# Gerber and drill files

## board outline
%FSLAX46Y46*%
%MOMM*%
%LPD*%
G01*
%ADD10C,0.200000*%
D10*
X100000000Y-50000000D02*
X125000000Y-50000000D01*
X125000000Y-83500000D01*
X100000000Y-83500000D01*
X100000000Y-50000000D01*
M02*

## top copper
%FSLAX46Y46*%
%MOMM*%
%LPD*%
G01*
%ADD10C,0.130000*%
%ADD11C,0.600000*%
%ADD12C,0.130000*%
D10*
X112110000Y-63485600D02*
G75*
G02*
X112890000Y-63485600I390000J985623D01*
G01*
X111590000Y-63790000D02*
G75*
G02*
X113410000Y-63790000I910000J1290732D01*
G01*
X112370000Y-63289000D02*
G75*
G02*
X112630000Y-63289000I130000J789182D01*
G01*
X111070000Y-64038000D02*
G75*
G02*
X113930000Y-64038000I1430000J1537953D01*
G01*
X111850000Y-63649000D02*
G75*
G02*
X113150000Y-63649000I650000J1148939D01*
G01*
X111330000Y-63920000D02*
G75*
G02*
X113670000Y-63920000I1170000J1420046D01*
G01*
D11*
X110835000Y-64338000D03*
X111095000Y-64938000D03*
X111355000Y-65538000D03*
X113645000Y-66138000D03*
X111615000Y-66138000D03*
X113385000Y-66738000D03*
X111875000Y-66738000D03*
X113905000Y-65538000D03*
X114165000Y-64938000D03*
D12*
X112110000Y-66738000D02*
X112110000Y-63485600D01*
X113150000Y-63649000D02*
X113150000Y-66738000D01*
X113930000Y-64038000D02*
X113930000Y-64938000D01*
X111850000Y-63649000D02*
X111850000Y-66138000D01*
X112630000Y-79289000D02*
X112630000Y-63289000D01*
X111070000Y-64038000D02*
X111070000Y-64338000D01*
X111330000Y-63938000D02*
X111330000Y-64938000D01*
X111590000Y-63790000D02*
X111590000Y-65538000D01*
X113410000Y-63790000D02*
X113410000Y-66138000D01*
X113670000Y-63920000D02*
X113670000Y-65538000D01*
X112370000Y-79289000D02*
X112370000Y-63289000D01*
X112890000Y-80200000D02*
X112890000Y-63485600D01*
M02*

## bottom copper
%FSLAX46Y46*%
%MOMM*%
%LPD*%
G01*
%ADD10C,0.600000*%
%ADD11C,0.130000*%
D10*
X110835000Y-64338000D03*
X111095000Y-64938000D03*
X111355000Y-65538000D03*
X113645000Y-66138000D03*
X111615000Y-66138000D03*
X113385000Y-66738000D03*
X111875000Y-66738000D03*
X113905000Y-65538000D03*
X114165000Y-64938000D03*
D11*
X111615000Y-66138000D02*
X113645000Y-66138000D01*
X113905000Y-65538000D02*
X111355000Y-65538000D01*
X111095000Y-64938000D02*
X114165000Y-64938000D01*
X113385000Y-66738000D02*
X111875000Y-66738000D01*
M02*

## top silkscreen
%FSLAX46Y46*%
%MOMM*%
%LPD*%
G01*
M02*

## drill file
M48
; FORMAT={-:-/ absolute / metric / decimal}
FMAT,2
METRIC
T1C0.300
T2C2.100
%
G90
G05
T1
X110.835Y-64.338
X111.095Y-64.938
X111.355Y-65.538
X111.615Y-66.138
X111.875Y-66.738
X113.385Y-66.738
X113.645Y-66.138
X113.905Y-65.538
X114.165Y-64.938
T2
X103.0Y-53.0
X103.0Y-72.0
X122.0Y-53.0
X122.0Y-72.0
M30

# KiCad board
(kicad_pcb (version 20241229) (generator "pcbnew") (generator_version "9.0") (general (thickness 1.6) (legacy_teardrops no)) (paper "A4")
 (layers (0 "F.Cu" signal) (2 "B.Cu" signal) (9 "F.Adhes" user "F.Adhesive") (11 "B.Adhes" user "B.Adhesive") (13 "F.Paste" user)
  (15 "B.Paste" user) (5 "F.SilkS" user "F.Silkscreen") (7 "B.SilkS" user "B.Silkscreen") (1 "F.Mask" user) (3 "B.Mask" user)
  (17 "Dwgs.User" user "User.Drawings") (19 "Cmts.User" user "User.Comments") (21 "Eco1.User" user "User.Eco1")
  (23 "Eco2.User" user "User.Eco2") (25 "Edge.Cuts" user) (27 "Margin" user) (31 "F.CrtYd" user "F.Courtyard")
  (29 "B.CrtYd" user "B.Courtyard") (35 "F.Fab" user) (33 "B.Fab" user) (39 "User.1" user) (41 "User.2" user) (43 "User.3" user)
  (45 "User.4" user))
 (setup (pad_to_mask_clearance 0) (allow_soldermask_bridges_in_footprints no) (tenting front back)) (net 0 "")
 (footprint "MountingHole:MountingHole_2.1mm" (layer "F.Cu") (at 122 53)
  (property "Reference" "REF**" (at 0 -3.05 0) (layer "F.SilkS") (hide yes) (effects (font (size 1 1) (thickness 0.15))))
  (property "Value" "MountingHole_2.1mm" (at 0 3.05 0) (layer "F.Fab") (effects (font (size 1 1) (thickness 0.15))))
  (pad "" np_thru_hole circle (at 0 0) (size 2.1 2.1) (drill 2.1) (layers "*.Cu" "*.Mask")))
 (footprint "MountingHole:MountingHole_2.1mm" (layer "F.Cu") (at 103 53)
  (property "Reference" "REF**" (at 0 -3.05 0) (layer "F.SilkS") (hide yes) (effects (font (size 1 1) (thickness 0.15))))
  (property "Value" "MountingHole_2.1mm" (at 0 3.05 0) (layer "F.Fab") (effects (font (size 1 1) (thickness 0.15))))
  (pad "" np_thru_hole circle (at 0 0) (size 2.1 2.1) (drill 2.1) (layers "*.Cu" "*.Mask")))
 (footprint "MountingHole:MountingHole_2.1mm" (layer "F.Cu") (at 103 72)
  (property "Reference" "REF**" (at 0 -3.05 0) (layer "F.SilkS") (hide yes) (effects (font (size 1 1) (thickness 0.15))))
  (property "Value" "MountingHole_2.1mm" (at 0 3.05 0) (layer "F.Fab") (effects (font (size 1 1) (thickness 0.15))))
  (pad "" np_thru_hole circle (at 0 0) (size 2.1 2.1) (drill 2.1) (layers "*.Cu" "*.Mask")))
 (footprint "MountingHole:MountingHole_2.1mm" (layer "F.Cu") (at 122 72)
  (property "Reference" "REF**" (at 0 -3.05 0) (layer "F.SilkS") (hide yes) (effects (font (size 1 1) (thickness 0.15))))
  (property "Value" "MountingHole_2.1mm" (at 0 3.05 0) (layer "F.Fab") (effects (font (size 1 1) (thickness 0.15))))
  (pad "" np_thru_hole circle (at 0 0) (size 2.1 2.1) (drill 2.1) (layers "*.Cu" "*.Mask")))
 (gr_arc (start 112.11 63.4856) (mid 112.5 61.44) (end 112.89 63.4856) (stroke (width 0.13) (type solid)) (layer "F.Cu"))
 (gr_arc (start 111.59 63.79) (mid 112.5 60.92) (end 113.41 63.79) (stroke (width 0.13) (type solid)) (layer "F.Cu"))
 (gr_arc (start 112.37 63.289) (mid 112.5 61.7) (end 112.63 63.289) (stroke (width 0.13) (type solid)) (layer "F.Cu"))
 (gr_arc (start 111.07 64.038) (mid 112.5 60.4) (end 113.93 64.038) (stroke (width 0.13) (type solid)) (layer "F.Cu"))
 (gr_arc (start 111.85 63.649) (mid 112.5 61.18) (end 113.15 63.649) (stroke (width 0.13) (type solid)) (layer "F.Cu"))
 (gr_arc (start 111.33 63.92) (mid 112.5 60.66) (end 113.67 63.92) (stroke (width 0.13) (type solid)) (layer "F.Cu"))
 (gr_rect (start 100 50) (end 125 83.5) (stroke (width 0.2) (type solid)) (fill no) (layer "Edge.Cuts"))
 (segment (start 112.11 66.738) (end 112.11 63.4856) (width 0.13) (layer "F.Cu") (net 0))
 (segment (start 113.15 63.649) (end 113.15 66.738) (width 0.13) (layer "F.Cu") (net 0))
 (segment (start 113.93 64.038) (end 113.93 64.938) (width 0.13) (layer "F.Cu") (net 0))
 (segment (start 111.85 63.649) (end 111.85 66.138) (width 0.13) (layer "F.Cu") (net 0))
 (segment (start 112.63 79.289) (end 112.63 63.289) (width 0.13) (layer "F.Cu") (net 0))
 (segment (start 111.07 64.038) (end 111.07 64.338) (width 0.13) (layer "F.Cu") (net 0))
 (segment (start 111.33 63.938) (end 111.33 64.938) (width 0.13) (layer "F.Cu") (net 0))
 (segment (start 111.59 63.79) (end 111.59 65.538) (width 0.13) (layer "F.Cu") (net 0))
 (segment (start 113.41 63.79) (end 113.41 66.138) (width 0.13) (layer "F.Cu") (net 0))
 (segment (start 113.67 63.92) (end 113.67 65.538) (width 0.13) (layer "F.Cu") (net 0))
 (segment (start 112.37 79.289) (end 112.37 63.289) (width 0.13) (layer "F.Cu") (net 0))
 (segment (start 112.89 80.2) (end 112.89 63.4856) (width 0.13) (layer "F.Cu") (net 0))
 (via (at 110.835 64.338) (size 0.6) (drill 0.3) (layers "F.Cu" "B.Cu") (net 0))
 (via (at 111.095 64.938) (size 0.6) (drill 0.3) (layers "F.Cu" "B.Cu") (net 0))
 (via (at 111.355 65.538) (size 0.6) (drill 0.3) (layers "F.Cu" "B.Cu") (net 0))
 (via (at 113.645 66.138) (size 0.6) (drill 0.3) (layers "F.Cu" "B.Cu") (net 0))
 (via (at 111.615 66.138) (size 0.6) (drill 0.3) (layers "F.Cu" "B.Cu") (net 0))
 (via (at 113.385 66.738) (size 0.6) (drill 0.3) (layers "F.Cu" "B.Cu") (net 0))
 (via (at 111.875 66.738) (size 0.6) (drill 0.3) (layers "F.Cu" "B.Cu") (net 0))
 (via (at 113.905 65.538) (size 0.6) (drill 0.3) (layers "F.Cu" "B.Cu") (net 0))
 (via (at 114.165 64.938) (size 0.6) (drill 0.3) (layers "F.Cu" "B.Cu") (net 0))
 (segment (start 111.615 66.138) (end 113.645 66.138) (width 0.13) (layer "B.Cu") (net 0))
 (segment (start 113.905 65.538) (end 111.355 65.538) (width 0.13) (layer "B.Cu") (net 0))
 (segment (start 111.095 64.938) (end 114.165 64.938) (width 0.13) (layer "B.Cu") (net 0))
 (segment (start 113.385 66.738) (end 111.875 66.738) (width 0.13) (layer "B.Cu") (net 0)))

